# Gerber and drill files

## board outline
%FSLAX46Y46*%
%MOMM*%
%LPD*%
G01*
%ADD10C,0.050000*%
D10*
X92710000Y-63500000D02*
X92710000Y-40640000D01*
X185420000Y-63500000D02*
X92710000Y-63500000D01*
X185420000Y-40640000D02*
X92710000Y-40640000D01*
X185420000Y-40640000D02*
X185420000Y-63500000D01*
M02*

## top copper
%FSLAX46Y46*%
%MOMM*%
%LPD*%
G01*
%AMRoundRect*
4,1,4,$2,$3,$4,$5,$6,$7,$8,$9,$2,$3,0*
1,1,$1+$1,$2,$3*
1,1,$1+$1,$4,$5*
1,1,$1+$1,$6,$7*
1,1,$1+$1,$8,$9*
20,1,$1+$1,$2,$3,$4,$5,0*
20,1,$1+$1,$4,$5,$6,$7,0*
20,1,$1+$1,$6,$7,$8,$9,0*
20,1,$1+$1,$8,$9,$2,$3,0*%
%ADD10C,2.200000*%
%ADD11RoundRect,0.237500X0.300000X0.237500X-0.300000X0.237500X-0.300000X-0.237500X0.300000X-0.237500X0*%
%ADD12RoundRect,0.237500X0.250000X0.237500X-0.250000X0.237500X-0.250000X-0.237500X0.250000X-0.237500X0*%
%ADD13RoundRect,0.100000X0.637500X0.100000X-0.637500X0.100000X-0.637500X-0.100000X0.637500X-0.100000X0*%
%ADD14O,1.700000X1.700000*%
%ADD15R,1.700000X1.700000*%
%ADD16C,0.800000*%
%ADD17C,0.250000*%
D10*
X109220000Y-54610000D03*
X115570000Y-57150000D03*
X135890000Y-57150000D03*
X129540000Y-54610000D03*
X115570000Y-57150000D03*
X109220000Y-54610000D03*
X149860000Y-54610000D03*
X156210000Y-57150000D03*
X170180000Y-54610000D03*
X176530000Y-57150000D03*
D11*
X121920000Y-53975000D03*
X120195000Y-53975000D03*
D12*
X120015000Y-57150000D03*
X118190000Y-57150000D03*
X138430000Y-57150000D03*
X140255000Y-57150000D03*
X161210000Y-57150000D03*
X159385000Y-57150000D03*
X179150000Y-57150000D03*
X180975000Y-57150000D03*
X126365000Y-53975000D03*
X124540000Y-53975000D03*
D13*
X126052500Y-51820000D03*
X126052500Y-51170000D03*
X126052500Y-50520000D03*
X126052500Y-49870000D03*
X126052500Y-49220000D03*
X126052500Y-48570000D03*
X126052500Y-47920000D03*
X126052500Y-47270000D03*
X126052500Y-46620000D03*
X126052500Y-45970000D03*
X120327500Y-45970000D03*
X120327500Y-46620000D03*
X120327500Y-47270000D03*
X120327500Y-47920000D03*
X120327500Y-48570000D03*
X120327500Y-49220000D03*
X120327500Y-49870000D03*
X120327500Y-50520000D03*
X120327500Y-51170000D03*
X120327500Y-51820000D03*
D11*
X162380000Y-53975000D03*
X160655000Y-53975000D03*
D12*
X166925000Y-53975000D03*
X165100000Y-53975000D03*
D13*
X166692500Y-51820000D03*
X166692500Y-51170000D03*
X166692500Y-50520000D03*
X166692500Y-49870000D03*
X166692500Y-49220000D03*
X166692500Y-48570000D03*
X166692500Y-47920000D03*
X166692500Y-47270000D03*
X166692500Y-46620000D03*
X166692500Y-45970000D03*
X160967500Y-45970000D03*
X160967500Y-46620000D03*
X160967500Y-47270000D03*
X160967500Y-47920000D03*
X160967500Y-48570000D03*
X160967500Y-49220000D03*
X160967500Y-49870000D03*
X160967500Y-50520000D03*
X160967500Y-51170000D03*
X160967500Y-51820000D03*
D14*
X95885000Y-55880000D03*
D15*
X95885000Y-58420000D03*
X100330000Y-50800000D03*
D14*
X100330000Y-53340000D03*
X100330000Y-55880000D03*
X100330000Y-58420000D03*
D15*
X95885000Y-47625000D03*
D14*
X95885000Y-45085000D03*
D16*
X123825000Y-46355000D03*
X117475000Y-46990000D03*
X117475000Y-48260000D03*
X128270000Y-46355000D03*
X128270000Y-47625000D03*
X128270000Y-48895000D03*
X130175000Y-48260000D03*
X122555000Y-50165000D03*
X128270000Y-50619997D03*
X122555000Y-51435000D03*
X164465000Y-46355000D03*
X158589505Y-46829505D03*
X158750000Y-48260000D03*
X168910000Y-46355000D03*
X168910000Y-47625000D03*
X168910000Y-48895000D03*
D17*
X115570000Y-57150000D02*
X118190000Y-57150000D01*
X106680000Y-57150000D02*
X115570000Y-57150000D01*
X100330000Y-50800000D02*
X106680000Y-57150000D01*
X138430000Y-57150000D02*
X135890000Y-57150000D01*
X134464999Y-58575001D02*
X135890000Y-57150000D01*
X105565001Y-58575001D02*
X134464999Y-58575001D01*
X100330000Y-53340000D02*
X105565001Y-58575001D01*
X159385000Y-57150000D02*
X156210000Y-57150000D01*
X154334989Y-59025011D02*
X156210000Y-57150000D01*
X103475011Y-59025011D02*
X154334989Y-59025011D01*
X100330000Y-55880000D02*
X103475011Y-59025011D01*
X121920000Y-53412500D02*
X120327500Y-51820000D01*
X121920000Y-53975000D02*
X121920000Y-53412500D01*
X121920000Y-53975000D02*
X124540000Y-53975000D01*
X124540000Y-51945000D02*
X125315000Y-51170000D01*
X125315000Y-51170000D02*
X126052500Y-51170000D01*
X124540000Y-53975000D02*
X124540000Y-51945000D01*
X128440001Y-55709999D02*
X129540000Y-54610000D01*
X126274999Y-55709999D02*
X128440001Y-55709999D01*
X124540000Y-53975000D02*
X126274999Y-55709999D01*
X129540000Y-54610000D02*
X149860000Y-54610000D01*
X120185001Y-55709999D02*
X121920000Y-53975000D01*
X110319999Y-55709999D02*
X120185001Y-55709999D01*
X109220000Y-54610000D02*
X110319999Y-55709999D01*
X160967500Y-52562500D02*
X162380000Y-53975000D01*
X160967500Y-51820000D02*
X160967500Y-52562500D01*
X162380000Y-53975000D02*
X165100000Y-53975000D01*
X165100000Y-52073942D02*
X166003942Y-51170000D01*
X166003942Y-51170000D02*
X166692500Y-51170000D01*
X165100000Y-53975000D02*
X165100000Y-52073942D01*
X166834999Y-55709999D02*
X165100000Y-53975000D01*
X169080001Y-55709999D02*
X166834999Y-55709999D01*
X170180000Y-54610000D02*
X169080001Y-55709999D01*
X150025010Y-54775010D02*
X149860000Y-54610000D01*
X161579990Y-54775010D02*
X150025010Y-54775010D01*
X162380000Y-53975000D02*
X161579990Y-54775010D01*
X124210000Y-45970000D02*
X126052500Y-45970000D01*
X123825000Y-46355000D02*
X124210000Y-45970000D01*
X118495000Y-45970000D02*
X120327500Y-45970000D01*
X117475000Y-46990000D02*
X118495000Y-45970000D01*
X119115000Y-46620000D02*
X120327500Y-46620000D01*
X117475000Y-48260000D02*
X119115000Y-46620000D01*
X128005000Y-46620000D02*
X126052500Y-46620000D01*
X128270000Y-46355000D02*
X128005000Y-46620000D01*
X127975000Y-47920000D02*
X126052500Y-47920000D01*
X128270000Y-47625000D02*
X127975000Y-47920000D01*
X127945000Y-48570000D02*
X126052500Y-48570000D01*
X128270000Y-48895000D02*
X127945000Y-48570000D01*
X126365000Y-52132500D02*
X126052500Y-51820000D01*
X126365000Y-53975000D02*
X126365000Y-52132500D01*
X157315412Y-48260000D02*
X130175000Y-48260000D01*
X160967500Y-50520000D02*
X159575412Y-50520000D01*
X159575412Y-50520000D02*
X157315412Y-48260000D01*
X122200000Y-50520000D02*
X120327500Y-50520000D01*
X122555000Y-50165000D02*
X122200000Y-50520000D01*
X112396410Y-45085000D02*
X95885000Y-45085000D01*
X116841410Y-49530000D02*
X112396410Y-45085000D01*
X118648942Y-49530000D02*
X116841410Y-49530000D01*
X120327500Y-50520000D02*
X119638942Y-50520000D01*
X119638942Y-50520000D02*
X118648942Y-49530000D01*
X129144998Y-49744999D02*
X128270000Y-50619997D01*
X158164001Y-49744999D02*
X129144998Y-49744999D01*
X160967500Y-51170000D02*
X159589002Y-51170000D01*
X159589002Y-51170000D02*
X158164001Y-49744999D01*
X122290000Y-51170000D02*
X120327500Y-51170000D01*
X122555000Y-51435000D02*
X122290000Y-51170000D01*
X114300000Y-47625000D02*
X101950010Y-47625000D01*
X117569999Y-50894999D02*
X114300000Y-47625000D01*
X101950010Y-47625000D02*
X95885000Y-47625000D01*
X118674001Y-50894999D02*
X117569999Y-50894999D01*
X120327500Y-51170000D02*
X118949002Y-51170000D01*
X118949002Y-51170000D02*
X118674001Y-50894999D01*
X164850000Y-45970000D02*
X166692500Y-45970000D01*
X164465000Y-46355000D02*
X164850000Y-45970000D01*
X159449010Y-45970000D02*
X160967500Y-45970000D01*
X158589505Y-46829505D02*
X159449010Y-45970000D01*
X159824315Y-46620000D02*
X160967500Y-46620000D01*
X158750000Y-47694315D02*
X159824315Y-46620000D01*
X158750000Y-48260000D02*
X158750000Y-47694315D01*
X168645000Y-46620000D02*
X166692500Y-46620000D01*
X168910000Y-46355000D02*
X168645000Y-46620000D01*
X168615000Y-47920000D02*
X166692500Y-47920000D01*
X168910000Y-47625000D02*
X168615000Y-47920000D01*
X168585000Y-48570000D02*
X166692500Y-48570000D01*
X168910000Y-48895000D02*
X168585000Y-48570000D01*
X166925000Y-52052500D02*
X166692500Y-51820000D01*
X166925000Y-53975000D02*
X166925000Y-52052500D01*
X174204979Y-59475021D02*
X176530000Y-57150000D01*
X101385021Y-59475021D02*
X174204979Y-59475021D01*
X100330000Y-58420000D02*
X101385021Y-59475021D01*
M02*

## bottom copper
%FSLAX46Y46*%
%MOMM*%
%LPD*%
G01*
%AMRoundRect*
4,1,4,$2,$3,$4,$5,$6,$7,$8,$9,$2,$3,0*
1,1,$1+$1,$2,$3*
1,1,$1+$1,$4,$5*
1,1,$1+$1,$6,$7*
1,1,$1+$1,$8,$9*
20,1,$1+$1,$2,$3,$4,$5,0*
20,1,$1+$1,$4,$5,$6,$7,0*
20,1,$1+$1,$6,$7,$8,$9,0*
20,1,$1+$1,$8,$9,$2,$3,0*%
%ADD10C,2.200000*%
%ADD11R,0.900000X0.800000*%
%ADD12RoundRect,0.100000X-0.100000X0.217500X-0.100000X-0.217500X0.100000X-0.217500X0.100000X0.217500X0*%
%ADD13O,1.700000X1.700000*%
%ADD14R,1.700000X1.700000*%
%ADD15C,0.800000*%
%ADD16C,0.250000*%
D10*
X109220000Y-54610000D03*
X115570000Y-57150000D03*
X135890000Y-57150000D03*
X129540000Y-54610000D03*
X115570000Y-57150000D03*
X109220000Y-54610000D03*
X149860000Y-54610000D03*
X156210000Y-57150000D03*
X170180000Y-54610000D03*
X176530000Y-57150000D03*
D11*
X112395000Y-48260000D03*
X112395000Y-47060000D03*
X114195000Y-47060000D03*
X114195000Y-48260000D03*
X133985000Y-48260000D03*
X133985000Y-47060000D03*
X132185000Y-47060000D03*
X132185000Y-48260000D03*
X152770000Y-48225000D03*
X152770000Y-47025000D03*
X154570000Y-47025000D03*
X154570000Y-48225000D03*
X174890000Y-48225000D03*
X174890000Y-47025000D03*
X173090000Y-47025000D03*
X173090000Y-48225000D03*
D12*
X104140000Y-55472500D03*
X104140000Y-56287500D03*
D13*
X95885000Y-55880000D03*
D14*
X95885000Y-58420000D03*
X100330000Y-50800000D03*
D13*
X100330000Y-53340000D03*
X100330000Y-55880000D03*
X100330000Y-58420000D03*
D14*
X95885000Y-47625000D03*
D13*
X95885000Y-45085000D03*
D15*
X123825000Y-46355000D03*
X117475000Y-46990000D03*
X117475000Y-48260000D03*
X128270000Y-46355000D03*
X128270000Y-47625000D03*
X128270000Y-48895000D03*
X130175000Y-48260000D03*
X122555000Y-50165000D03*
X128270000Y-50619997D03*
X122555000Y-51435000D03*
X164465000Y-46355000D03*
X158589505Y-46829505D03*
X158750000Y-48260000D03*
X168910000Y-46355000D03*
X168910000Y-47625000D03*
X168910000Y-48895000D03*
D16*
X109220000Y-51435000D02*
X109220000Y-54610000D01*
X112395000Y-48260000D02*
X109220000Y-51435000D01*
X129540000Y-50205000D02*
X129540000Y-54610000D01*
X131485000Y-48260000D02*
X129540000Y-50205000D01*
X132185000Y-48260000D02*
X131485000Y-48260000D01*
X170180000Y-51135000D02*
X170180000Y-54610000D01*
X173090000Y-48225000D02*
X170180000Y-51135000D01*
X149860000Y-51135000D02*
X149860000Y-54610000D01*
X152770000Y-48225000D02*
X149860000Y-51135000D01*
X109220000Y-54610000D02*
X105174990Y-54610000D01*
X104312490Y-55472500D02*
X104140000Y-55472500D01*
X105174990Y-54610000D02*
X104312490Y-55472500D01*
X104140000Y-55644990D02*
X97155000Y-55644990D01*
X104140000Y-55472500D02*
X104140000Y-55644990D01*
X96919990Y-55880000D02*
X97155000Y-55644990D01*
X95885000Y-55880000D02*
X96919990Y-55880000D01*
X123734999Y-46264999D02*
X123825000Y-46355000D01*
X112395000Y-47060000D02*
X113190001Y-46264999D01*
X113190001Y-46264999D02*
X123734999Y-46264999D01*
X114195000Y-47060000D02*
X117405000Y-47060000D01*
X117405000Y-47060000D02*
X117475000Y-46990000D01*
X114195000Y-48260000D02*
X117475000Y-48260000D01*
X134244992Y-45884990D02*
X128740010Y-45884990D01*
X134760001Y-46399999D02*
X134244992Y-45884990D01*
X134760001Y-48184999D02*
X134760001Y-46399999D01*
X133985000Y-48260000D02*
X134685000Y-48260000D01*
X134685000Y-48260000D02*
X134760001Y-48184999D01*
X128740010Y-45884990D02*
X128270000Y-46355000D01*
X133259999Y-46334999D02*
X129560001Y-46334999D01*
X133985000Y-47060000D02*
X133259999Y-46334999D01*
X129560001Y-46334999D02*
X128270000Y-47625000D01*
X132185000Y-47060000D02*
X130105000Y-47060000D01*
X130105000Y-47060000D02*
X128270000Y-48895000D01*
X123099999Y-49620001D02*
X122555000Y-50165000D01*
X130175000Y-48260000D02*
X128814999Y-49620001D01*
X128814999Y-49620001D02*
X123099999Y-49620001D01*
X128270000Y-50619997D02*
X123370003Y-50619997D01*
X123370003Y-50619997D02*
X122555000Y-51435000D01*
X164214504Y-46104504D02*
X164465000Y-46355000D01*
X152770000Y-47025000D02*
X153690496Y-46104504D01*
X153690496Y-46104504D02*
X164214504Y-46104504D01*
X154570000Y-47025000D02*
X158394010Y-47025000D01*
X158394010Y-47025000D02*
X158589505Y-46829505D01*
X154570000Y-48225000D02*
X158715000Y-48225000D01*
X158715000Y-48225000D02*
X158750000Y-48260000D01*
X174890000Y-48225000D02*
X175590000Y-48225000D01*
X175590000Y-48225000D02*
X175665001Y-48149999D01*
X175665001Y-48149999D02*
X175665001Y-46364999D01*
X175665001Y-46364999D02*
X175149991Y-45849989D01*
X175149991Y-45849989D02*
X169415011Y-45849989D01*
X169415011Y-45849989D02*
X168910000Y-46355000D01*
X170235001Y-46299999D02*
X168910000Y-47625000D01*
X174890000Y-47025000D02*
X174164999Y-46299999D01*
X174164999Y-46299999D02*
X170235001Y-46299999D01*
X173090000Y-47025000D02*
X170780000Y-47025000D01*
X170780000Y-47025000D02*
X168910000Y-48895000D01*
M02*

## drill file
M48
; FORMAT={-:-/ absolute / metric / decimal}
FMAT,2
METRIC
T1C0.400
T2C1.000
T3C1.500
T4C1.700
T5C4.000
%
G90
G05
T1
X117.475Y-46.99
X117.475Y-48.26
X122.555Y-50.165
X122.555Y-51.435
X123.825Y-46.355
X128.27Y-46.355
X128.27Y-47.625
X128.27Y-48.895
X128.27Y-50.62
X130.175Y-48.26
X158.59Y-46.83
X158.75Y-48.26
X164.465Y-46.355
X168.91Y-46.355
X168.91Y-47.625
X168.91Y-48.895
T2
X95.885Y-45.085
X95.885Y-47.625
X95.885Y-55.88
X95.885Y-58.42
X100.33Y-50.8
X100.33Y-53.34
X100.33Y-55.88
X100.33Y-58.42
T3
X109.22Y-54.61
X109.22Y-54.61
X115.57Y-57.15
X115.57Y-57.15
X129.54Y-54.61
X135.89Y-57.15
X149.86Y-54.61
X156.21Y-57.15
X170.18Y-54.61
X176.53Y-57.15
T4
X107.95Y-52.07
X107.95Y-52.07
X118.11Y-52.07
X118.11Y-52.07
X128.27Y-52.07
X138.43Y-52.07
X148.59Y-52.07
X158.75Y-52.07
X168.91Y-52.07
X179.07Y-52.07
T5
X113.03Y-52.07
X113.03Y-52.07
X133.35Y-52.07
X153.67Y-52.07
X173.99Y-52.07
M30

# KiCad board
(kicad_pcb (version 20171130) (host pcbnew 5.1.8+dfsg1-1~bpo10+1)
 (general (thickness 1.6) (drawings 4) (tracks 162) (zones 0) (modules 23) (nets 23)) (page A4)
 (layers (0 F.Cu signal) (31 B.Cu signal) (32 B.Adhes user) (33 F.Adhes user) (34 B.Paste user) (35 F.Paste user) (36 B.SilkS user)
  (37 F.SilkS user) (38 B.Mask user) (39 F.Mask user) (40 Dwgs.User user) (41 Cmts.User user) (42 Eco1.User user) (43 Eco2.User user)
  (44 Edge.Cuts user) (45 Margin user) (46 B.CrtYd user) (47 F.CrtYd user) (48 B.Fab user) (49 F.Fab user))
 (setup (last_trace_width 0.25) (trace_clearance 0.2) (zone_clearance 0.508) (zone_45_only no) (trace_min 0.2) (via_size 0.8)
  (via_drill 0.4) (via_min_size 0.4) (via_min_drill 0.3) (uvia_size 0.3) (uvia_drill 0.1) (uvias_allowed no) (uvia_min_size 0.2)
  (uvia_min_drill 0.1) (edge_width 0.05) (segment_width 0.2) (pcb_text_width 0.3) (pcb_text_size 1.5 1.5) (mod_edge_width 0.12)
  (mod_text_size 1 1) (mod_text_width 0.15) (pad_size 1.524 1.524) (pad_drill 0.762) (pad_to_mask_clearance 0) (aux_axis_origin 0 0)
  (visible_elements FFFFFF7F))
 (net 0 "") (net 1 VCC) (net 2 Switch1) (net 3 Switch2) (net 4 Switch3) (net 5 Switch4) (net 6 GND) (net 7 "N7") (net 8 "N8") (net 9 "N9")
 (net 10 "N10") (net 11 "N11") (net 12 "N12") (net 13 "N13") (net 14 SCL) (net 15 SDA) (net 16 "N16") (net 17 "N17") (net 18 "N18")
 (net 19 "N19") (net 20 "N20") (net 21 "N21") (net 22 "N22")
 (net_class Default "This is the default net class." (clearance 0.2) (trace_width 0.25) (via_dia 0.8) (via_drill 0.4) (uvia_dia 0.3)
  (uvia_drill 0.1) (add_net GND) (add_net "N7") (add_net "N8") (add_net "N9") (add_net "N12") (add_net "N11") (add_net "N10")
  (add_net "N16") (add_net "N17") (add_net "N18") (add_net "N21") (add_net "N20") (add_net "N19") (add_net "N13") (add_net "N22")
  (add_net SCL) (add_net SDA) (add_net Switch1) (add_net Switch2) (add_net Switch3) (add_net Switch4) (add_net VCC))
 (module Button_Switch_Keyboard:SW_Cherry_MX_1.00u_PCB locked (layer B.Cu) (at 115.57 57.15)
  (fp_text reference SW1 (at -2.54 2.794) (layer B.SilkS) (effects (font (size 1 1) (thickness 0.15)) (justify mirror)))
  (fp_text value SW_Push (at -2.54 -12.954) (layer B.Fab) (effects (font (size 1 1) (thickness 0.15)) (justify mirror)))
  (pad "" np_thru_hole circle (at 2.54 -5.08) (size 1.7 1.7) (drill 1.7) (layers *.Cu *.Mask))
  (pad "" np_thru_hole circle (at -7.62 -5.08) (size 1.7 1.7) (drill 1.7) (layers *.Cu *.Mask))
  (pad "" np_thru_hole circle (at -2.54 -5.08) (size 4 4) (drill 4) (layers *.Cu *.Mask))
  (pad 2 thru_hole circle (at -6.35 -2.54) (size 2.2 2.2) (drill 1.5) (layers *.Cu *.Mask) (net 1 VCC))
  (pad 1 thru_hole circle (at 0 0) (size 2.2 2.2) (drill 1.5) (layers *.Cu *.Mask) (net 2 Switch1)))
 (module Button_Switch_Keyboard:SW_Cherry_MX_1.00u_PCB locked (layer B.Cu) (at 135.89 57.15)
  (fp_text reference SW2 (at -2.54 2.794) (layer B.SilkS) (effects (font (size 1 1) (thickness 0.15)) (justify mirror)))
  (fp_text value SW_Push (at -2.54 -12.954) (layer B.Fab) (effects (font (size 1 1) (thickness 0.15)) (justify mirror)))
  (pad 1 thru_hole circle (at 0 0) (size 2.2 2.2) (drill 1.5) (layers *.Cu *.Mask) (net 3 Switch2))
  (pad 2 thru_hole circle (at -6.35 -2.54) (size 2.2 2.2) (drill 1.5) (layers *.Cu *.Mask) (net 1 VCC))
  (pad "" np_thru_hole circle (at -2.54 -5.08) (size 4 4) (drill 4) (layers *.Cu *.Mask))
  (pad "" np_thru_hole circle (at -7.62 -5.08) (size 1.7 1.7) (drill 1.7) (layers *.Cu *.Mask))
  (pad "" np_thru_hole circle (at 2.54 -5.08) (size 1.7 1.7) (drill 1.7) (layers *.Cu *.Mask)))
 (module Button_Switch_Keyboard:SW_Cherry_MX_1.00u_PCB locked (layer B.Cu) (at 115.57 57.15)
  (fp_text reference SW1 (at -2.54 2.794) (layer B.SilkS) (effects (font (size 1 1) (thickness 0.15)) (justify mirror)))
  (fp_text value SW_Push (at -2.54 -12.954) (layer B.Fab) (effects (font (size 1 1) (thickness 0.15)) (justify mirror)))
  (pad 1 thru_hole circle (at 0 0) (size 2.2 2.2) (drill 1.5) (layers *.Cu *.Mask) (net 2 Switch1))
  (pad 2 thru_hole circle (at -6.35 -2.54) (size 2.2 2.2) (drill 1.5) (layers *.Cu *.Mask) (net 1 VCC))
  (pad "" np_thru_hole circle (at -2.54 -5.08) (size 4 4) (drill 4) (layers *.Cu *.Mask))
  (pad "" np_thru_hole circle (at -7.62 -5.08) (size 1.7 1.7) (drill 1.7) (layers *.Cu *.Mask))
  (pad "" np_thru_hole circle (at 2.54 -5.08) (size 1.7 1.7) (drill 1.7) (layers *.Cu *.Mask)))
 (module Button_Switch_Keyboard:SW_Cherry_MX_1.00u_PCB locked (layer B.Cu) (at 156.21 57.15)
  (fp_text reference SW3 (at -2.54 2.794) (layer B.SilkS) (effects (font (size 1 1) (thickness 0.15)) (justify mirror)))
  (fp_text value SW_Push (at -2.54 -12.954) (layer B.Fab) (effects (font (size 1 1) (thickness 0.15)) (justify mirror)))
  (pad "" np_thru_hole circle (at 2.54 -5.08) (size 1.7 1.7) (drill 1.7) (layers *.Cu *.Mask))
  (pad "" np_thru_hole circle (at -7.62 -5.08) (size 1.7 1.7) (drill 1.7) (layers *.Cu *.Mask))
  (pad "" np_thru_hole circle (at -2.54 -5.08) (size 4 4) (drill 4) (layers *.Cu *.Mask))
  (pad 2 thru_hole circle (at -6.35 -2.54) (size 2.2 2.2) (drill 1.5) (layers *.Cu *.Mask) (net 1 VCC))
  (pad 1 thru_hole circle (at 0 0) (size 2.2 2.2) (drill 1.5) (layers *.Cu *.Mask) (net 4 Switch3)))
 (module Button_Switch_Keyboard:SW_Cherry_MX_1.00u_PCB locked (layer B.Cu) (at 176.53 57.15)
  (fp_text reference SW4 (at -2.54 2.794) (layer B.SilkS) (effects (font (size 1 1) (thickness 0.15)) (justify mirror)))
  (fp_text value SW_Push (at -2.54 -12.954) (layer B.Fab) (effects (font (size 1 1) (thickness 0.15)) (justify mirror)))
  (pad "" np_thru_hole circle (at 2.54 -5.08) (size 1.7 1.7) (drill 1.7) (layers *.Cu *.Mask))
  (pad "" np_thru_hole circle (at -7.62 -5.08) (size 1.7 1.7) (drill 1.7) (layers *.Cu *.Mask))
  (pad "" np_thru_hole circle (at -2.54 -5.08) (size 4 4) (drill 4) (layers *.Cu *.Mask))
  (pad 2 thru_hole circle (at -6.35 -2.54) (size 2.2 2.2) (drill 1.5) (layers *.Cu *.Mask) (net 1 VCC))
  (pad 1 thru_hole circle (at 0 0) (size 2.2 2.2) (drill 1.5) (layers *.Cu *.Mask) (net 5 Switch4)))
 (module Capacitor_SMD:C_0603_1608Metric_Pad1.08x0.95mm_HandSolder (layer F.Cu) (at 121.0575 53.975 180)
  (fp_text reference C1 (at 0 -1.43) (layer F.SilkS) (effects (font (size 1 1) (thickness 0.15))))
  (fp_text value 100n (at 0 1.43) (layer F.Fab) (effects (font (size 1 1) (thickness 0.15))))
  (pad 1 smd roundrect (at -0.8625 0 180) (size 1.075 0.95) (layers F.Cu F.Paste F.Mask) (roundrect_rratio 0.25) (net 1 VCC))
  (pad 2 smd roundrect (at 0.8625 0 180) (size 1.075 0.95) (layers F.Cu F.Paste F.Mask) (roundrect_rratio 0.25) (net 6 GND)))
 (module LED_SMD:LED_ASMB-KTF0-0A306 (layer B.Cu) (at 113.295 47.66)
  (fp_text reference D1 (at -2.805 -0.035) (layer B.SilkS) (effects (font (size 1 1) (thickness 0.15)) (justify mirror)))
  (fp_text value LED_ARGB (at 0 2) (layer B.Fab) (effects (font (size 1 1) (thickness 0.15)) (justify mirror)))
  (pad 1 smd rect (at -0.9 0.6) (size 0.9 0.8) (layers B.Cu B.Paste B.Mask) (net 1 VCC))
  (pad 2 smd rect (at -0.9 -0.6) (size 0.9 0.8) (layers B.Cu B.Paste B.Mask) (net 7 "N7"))
  (pad 3 smd rect (at 0.9 -0.6) (size 0.9 0.8) (layers B.Cu B.Paste B.Mask) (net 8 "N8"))
  (pad 4 smd rect (at 0.9 0.6) (size 0.9 0.8) (layers B.Cu B.Paste B.Mask) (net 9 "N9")))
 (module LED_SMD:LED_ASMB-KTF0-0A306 (layer B.Cu) (at 133.085 47.66)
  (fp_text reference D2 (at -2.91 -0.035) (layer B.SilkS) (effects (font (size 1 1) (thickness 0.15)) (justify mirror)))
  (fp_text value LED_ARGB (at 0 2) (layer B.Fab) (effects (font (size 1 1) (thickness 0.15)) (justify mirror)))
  (pad 4 smd rect (at 0.9 0.6) (size 0.9 0.8) (layers B.Cu B.Paste B.Mask) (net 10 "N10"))
  (pad 3 smd rect (at 0.9 -0.6) (size 0.9 0.8) (layers B.Cu B.Paste B.Mask) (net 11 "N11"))
  (pad 2 smd rect (at -0.9 -0.6) (size 0.9 0.8) (layers B.Cu B.Paste B.Mask) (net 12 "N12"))
  (pad 1 smd rect (at -0.9 0.6) (size 0.9 0.8) (layers B.Cu B.Paste B.Mask) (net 1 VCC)))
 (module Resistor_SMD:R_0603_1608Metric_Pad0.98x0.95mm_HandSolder (layer F.Cu) (at 119.1025 57.15 180)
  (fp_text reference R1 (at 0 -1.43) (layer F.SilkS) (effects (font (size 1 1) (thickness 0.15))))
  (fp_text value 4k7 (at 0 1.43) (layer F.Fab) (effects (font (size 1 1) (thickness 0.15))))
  (pad 1 smd roundrect (at -0.9125 0 180) (size 0.975 0.95) (layers F.Cu F.Paste F.Mask) (roundrect_rratio 0.25) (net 6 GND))
  (pad 2 smd roundrect (at 0.9125 0 180) (size 0.975 0.95) (layers F.Cu F.Paste F.Mask) (roundrect_rratio 0.25) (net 2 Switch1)))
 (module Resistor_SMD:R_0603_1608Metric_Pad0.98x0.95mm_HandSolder (layer F.Cu) (at 139.3425 57.15 180)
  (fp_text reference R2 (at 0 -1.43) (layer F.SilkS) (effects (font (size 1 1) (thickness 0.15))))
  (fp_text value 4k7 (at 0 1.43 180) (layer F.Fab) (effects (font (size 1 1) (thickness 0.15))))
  (pad 2 smd roundrect (at 0.9125 0 180) (size 0.975 0.95) (layers F.Cu F.Paste F.Mask) (roundrect_rratio 0.25) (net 3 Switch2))
  (pad 1 smd roundrect (at -0.9125 0 180) (size 0.975 0.95) (layers F.Cu F.Paste F.Mask) (roundrect_rratio 0.25) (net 6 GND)))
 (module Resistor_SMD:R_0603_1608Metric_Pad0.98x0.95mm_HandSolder (layer F.Cu) (at 160.2975 57.15 180)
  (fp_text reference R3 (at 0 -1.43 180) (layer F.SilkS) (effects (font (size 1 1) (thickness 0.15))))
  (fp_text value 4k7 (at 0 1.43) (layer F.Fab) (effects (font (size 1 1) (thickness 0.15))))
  (pad 1 smd roundrect (at -0.9125 0 180) (size 0.975 0.95) (layers F.Cu F.Paste F.Mask) (roundrect_rratio 0.25) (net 6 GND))
  (pad 2 smd roundrect (at 0.9125 0 180) (size 0.975 0.95) (layers F.Cu F.Paste F.Mask) (roundrect_rratio 0.25) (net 4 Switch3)))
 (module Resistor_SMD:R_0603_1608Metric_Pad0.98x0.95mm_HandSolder (layer F.Cu) (at 180.0625 57.15 180)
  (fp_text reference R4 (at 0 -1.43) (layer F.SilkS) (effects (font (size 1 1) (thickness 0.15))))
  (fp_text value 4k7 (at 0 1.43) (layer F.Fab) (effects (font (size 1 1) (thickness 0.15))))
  (pad 2 smd roundrect (at 0.9125 0 180) (size 0.975 0.95) (layers F.Cu F.Paste F.Mask) (roundrect_rratio 0.25))
  (pad 1 smd roundrect (at -0.9125 0 180) (size 0.975 0.95) (layers F.Cu F.Paste F.Mask) (roundrect_rratio 0.25) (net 6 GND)))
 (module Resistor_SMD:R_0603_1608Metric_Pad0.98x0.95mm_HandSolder (layer F.Cu) (at 125.4525 53.975 180)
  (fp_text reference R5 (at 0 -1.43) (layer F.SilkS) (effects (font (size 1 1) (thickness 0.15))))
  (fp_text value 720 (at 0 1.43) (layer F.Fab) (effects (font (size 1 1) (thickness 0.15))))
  (pad 1 smd roundrect (at -0.9125 0 180) (size 0.975 0.95) (layers F.Cu F.Paste F.Mask) (roundrect_rratio 0.25) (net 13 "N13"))
  (pad 2 smd roundrect (at 0.9125 0 180) (size 0.975 0.95) (layers F.Cu F.Paste F.Mask) (roundrect_rratio 0.25) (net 1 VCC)))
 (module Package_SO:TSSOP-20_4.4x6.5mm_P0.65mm (layer F.Cu) (at 123.19 48.895 180)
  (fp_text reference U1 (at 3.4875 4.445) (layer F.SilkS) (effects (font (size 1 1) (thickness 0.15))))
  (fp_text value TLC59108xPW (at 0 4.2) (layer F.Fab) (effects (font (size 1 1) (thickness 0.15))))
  (pad 1 smd roundrect (at -2.8625 -2.925 180) (size 1.475 0.4) (layers F.Cu F.Paste F.Mask) (roundrect_rratio 0.25) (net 13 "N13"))
  (pad 2 smd roundrect (at -2.8625 -2.275 180) (size 1.475 0.4) (layers F.Cu F.Paste F.Mask) (roundrect_rratio 0.25) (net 1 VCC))
  (pad 3 smd roundrect (at -2.8625 -1.625 180) (size 1.475 0.4) (layers F.Cu F.Paste F.Mask) (roundrect_rratio 0.25) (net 6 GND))
  (pad 4 smd roundrect (at -2.8625 -0.975 180) (size 1.475 0.4) (layers F.Cu F.Paste F.Mask) (roundrect_rratio 0.25) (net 6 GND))
  (pad 5 smd roundrect (at -2.8625 -0.325 180) (size 1.475 0.4) (layers F.Cu F.Paste F.Mask) (roundrect_rratio 0.25) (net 6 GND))
  (pad 6 smd roundrect (at -2.8625 0.325 180) (size 1.475 0.4) (layers F.Cu F.Paste F.Mask) (roundrect_rratio 0.25) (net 12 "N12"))
  (pad 7 smd roundrect (at -2.8625 0.975 180) (size 1.475 0.4) (layers F.Cu F.Paste F.Mask) (roundrect_rratio 0.25) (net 11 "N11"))
  (pad 8 smd roundrect (at -2.8625 1.625 180) (size 1.475 0.4) (layers F.Cu F.Paste F.Mask) (roundrect_rratio 0.25) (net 6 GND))
  (pad 9 smd roundrect (at -2.8625 2.275 180) (size 1.475 0.4) (layers F.Cu F.Paste F.Mask) (roundrect_rratio 0.25) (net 10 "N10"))
  (pad 10 smd roundrect (at -2.8625 2.925 180) (size 1.475 0.4) (layers F.Cu F.Paste F.Mask) (roundrect_rratio 0.25) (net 7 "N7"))
  (pad 11 smd roundrect (at 2.8625 2.925 180) (size 1.475 0.4) (layers F.Cu F.Paste F.Mask) (roundrect_rratio 0.25) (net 8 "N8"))
  (pad 12 smd roundrect (at 2.8625 2.275 180) (size 1.475 0.4) (layers F.Cu F.Paste F.Mask) (roundrect_rratio 0.25) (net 9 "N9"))
  (pad 13 smd roundrect (at 2.8625 1.625 180) (size 1.475 0.4) (layers F.Cu F.Paste F.Mask) (roundrect_rratio 0.25) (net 6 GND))
  (pad 14 smd roundrect (at 2.8625 0.975 180) (size 1.475 0.4) (layers F.Cu F.Paste F.Mask) (roundrect_rratio 0.25))
  (pad 15 smd roundrect (at 2.8625 0.325 180) (size 1.475 0.4) (layers F.Cu F.Paste F.Mask) (roundrect_rratio 0.25))
  (pad 16 smd roundrect (at 2.8625 -0.325 180) (size 1.475 0.4) (layers F.Cu F.Paste F.Mask) (roundrect_rratio 0.25) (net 6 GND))
  (pad 17 smd roundrect (at 2.8625 -0.975 180) (size 1.475 0.4) (layers F.Cu F.Paste F.Mask) (roundrect_rratio 0.25) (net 1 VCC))
  (pad 18 smd roundrect (at 2.8625 -1.625 180) (size 1.475 0.4) (layers F.Cu F.Paste F.Mask) (roundrect_rratio 0.25) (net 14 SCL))
  (pad 19 smd roundrect (at 2.8625 -2.275 180) (size 1.475 0.4) (layers F.Cu F.Paste F.Mask) (roundrect_rratio 0.25) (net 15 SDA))
  (pad 20 smd roundrect (at 2.8625 -2.925 180) (size 1.475 0.4) (layers F.Cu F.Paste F.Mask) (roundrect_rratio 0.25) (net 1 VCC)))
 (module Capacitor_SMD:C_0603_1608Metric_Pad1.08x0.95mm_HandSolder (layer F.Cu) (at 161.5175 53.975 180)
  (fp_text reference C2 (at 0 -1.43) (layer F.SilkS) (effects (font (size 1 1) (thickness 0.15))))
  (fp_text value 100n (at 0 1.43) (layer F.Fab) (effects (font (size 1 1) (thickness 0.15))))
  (pad 1 smd roundrect (at -0.8625 0 180) (size 1.075 0.95) (layers F.Cu F.Paste F.Mask) (roundrect_rratio 0.25) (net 1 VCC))
  (pad 2 smd roundrect (at 0.8625 0 180) (size 1.075 0.95) (layers F.Cu F.Paste F.Mask) (roundrect_rratio 0.25) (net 6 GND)))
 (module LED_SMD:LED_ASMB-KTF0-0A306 (layer B.Cu) (at 153.67 47.625)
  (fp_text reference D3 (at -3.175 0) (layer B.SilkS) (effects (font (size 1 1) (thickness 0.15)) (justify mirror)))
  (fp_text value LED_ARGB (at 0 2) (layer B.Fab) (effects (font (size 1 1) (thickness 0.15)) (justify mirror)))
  (pad 1 smd rect (at -0.9 0.6) (size 0.9 0.8) (layers B.Cu B.Paste B.Mask) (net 1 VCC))
  (pad 2 smd rect (at -0.9 -0.6) (size 0.9 0.8) (layers B.Cu B.Paste B.Mask) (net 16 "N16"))
  (pad 3 smd rect (at 0.9 -0.6) (size 0.9 0.8) (layers B.Cu B.Paste B.Mask) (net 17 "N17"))
  (pad 4 smd rect (at 0.9 0.6) (size 0.9 0.8) (layers B.Cu B.Paste B.Mask) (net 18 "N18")))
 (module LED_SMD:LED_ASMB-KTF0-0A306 (layer B.Cu) (at 173.99 47.625)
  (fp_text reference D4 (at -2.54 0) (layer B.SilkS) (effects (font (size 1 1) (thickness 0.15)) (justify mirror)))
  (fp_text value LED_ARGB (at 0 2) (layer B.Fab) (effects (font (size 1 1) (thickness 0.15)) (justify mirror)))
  (pad 4 smd rect (at 0.9 0.6) (size 0.9 0.8) (layers B.Cu B.Paste B.Mask) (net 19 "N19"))
  (pad 3 smd rect (at 0.9 -0.6) (size 0.9 0.8) (layers B.Cu B.Paste B.Mask) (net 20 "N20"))
  (pad 2 smd rect (at -0.9 -0.6) (size 0.9 0.8) (layers B.Cu B.Paste B.Mask) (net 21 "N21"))
  (pad 1 smd rect (at -0.9 0.6) (size 0.9 0.8) (layers B.Cu B.Paste B.Mask) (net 1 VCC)))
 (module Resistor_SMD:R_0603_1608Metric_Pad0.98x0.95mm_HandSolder (layer F.Cu) (at 166.0125 53.975 180)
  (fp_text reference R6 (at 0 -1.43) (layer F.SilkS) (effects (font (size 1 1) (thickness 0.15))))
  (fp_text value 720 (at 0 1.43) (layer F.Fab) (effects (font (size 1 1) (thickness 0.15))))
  (pad 1 smd roundrect (at -0.9125 0 180) (size 0.975 0.95) (layers F.Cu F.Paste F.Mask) (roundrect_rratio 0.25) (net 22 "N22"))
  (pad 2 smd roundrect (at 0.9125 0 180) (size 0.975 0.95) (layers F.Cu F.Paste F.Mask) (roundrect_rratio 0.25) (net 1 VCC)))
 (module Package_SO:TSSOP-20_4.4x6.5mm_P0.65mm (layer F.Cu) (at 163.83 48.895 180)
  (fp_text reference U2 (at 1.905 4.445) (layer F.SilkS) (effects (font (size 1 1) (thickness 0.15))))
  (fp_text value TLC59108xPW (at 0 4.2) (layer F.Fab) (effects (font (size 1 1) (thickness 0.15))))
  (pad 1 smd roundrect (at -2.8625 -2.925 180) (size 1.475 0.4) (layers F.Cu F.Paste F.Mask) (roundrect_rratio 0.25) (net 22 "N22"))
  (pad 2 smd roundrect (at -2.8625 -2.275 180) (size 1.475 0.4) (layers F.Cu F.Paste F.Mask) (roundrect_rratio 0.25) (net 1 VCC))
  (pad 3 smd roundrect (at -2.8625 -1.625 180) (size 1.475 0.4) (layers F.Cu F.Paste F.Mask) (roundrect_rratio 0.25) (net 1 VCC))
  (pad 4 smd roundrect (at -2.8625 -0.975 180) (size 1.475 0.4) (layers F.Cu F.Paste F.Mask) (roundrect_rratio 0.25) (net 6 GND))
  (pad 5 smd roundrect (at -2.8625 -0.325 180) (size 1.475 0.4) (layers F.Cu F.Paste F.Mask) (roundrect_rratio 0.25) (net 6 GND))
  (pad 6 smd roundrect (at -2.8625 0.325 180) (size 1.475 0.4) (layers F.Cu F.Paste F.Mask) (roundrect_rratio 0.25) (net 21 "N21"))
  (pad 7 smd roundrect (at -2.8625 0.975 180) (size 1.475 0.4) (layers F.Cu F.Paste F.Mask) (roundrect_rratio 0.25) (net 20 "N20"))
  (pad 8 smd roundrect (at -2.8625 1.625 180) (size 1.475 0.4) (layers F.Cu F.Paste F.Mask) (roundrect_rratio 0.25) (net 6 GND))
  (pad 9 smd roundrect (at -2.8625 2.275 180) (size 1.475 0.4) (layers F.Cu F.Paste F.Mask) (roundrect_rratio 0.25) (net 19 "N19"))
  (pad 10 smd roundrect (at -2.8625 2.925 180) (size 1.475 0.4) (layers F.Cu F.Paste F.Mask) (roundrect_rratio 0.25) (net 16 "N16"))
  (pad 11 smd roundrect (at 2.8625 2.925 180) (size 1.475 0.4) (layers F.Cu F.Paste F.Mask) (roundrect_rratio 0.25) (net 17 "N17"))
  (pad 12 smd roundrect (at 2.8625 2.275 180) (size 1.475 0.4) (layers F.Cu F.Paste F.Mask) (roundrect_rratio 0.25) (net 18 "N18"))
  (pad 13 smd roundrect (at 2.8625 1.625 180) (size 1.475 0.4) (layers F.Cu F.Paste F.Mask) (roundrect_rratio 0.25) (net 6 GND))
  (pad 14 smd roundrect (at 2.8625 0.975 180) (size 1.475 0.4) (layers F.Cu F.Paste F.Mask) (roundrect_rratio 0.25))
  (pad 15 smd roundrect (at 2.8625 0.325 180) (size 1.475 0.4) (layers F.Cu F.Paste F.Mask) (roundrect_rratio 0.25))
  (pad 16 smd roundrect (at 2.8625 -0.325 180) (size 1.475 0.4) (layers F.Cu F.Paste F.Mask) (roundrect_rratio 0.25) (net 6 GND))
  (pad 17 smd roundrect (at 2.8625 -0.975 180) (size 1.475 0.4) (layers F.Cu F.Paste F.Mask) (roundrect_rratio 0.25) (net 1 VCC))
  (pad 18 smd roundrect (at 2.8625 -1.625 180) (size 1.475 0.4) (layers F.Cu F.Paste F.Mask) (roundrect_rratio 0.25) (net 14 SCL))
  (pad 19 smd roundrect (at 2.8625 -2.275 180) (size 1.475 0.4) (layers F.Cu F.Paste F.Mask) (roundrect_rratio 0.25) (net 15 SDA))
  (pad 20 smd roundrect (at 2.8625 -2.925 180) (size 1.475 0.4) (layers F.Cu F.Paste F.Mask) (roundrect_rratio 0.25) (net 1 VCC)))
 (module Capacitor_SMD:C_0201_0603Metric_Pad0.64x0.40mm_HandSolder (layer B.Cu) (at 104.14 55.88 270)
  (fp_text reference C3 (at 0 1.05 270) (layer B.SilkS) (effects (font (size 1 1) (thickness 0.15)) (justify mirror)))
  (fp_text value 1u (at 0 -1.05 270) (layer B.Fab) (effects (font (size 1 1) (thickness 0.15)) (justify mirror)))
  (pad "" smd roundrect (at -0.4325 0 270) (size 0.458 0.36) (layers B.Paste) (roundrect_rratio 0.25))
  (pad "" smd roundrect (at 0.4325 0 270) (size 0.458 0.36) (layers B.Paste) (roundrect_rratio 0.25))
  (pad 1 smd roundrect (at -0.4075 0 270) (size 0.635 0.4) (layers B.Cu B.Mask) (roundrect_rratio 0.25) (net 1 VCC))
  (pad 2 smd roundrect (at 0.4075 0 270) (size 0.635 0.4) (layers B.Cu B.Mask) (roundrect_rratio 0.25) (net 6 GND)))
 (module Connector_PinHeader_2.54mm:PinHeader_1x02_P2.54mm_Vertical (layer F.Cu) (at 95.885 58.42 180)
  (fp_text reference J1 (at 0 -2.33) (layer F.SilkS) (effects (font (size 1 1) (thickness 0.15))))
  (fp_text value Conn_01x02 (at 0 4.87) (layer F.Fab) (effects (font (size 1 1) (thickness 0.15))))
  (pad 2 thru_hole oval (at 0 2.54 180) (size 1.7 1.7) (drill 1) (layers *.Cu *.Mask) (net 1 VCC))
  (pad 1 thru_hole rect (at 0 0 180) (size 1.7 1.7) (drill 1) (layers *.Cu *.Mask) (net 6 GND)))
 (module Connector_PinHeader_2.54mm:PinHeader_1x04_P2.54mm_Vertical (layer B.Cu) (at 100.33 50.8 180)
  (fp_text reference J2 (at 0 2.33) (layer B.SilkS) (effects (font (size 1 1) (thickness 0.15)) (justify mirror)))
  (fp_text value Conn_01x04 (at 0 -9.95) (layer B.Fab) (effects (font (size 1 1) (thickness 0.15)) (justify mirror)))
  (pad 1 thru_hole rect (at 0 0 180) (size 1.7 1.7) (drill 1) (layers *.Cu *.Mask) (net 2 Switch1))
  (pad 2 thru_hole oval (at 0 -2.54 180) (size 1.7 1.7) (drill 1) (layers *.Cu *.Mask) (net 3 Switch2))
  (pad 3 thru_hole oval (at 0 -5.08 180) (size 1.7 1.7) (drill 1) (layers *.Cu *.Mask) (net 4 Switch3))
  (pad 4 thru_hole oval (at 0 -7.62 180) (size 1.7 1.7) (drill 1) (layers *.Cu *.Mask) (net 5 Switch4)))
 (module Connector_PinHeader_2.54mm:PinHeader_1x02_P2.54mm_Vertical (layer B.Cu) (at 95.885 47.625)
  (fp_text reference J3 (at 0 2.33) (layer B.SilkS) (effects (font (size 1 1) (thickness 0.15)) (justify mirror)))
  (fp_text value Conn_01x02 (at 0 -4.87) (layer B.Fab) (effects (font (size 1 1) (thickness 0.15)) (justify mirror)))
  (pad 1 thru_hole rect (at 0 0) (size 1.7 1.7) (drill 1) (layers *.Cu *.Mask) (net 15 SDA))
  (pad 2 thru_hole oval (at 0 -2.54) (size 1.7 1.7) (drill 1) (layers *.Cu *.Mask) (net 14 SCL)))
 (gr_line (start 92.71 63.5) (end 92.71 40.64) (layer Edge.Cuts) (width 0.05))
 (gr_line (start 185.42 63.5) (end 92.71 63.5) (layer Edge.Cuts) (width 0.05))
 (gr_line (start 185.42 40.64) (end 92.71 40.64) (layer Edge.Cuts) (width 0.05))
 (gr_line (start 185.42 40.64) (end 185.42 63.5) (layer Edge.Cuts) (width 0.05))
 (segment (start 115.57 57.15) (end 118.19 57.15) (width 0.25) (layer F.Cu) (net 2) (status 30))
 (segment (start 106.68 57.15) (end 115.57 57.15) (width 0.25) (layer F.Cu) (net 2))
 (segment (start 100.33 50.8) (end 106.68 57.15) (width 0.25) (layer F.Cu) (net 2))
 (segment (start 138.43 57.15) (end 135.89 57.15) (width 0.25) (layer F.Cu) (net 3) (status 30))
 (segment (start 134.464999 58.575001) (end 135.89 57.15) (width 0.25) (layer F.Cu) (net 3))
 (segment (start 105.565001 58.575001) (end 134.464999 58.575001) (width 0.25) (layer F.Cu) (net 3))
 (segment (start 100.33 53.34) (end 105.565001 58.575001) (width 0.25) (layer F.Cu) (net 3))
 (segment (start 159.385 57.15) (end 156.21 57.15) (width 0.25) (layer F.Cu) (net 4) (status 30))
 (segment (start 154.334989 59.025011) (end 156.21 57.15) (width 0.25) (layer F.Cu) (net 4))
 (segment (start 103.475011 59.025011) (end 154.334989 59.025011) (width 0.25) (layer F.Cu) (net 4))
 (segment (start 100.33 55.88) (end 103.475011 59.025011) (width 0.25) (layer F.Cu) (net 4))
 (segment (start 121.92 53.4125) (end 120.3275 51.82) (width 0.25) (layer F.Cu) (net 1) (status 20))
 (segment (start 121.92 53.975) (end 121.92 53.4125) (width 0.25) (layer F.Cu) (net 1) (status 10))
 (segment (start 121.92 53.975) (end 124.54 53.975) (width 0.25) (layer F.Cu) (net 1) (status 30))
 (segment (start 124.54 51.945) (end 125.315 51.17) (width 0.25) (layer F.Cu) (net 1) (status 20))
 (segment (start 125.315 51.17) (end 126.0525 51.17) (width 0.25) (layer F.Cu) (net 1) (status 30))
 (segment (start 124.54 53.975) (end 124.54 51.945) (width 0.25) (layer F.Cu) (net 1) (status 10))
 (segment (start 128.440001 55.709999) (end 129.54 54.61) (width 0.25) (layer F.Cu) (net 1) (status 20))
 (segment (start 126.274999 55.709999) (end 128.440001 55.709999) (width 0.25) (layer F.Cu) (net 1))
 (segment (start 124.54 53.975) (end 126.274999 55.709999) (width 0.25) (layer F.Cu) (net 1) (status 10))
 (segment (start 129.54 54.61) (end 149.86 54.61) (width 0.25) (layer F.Cu) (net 1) (status 30))
 (segment (start 120.185001 55.709999) (end 121.92 53.975) (width 0.25) (layer F.Cu) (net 1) (status 20))
 (segment (start 110.319999 55.709999) (end 120.185001 55.709999) (width 0.25) (layer F.Cu) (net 1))
 (segment (start 109.22 54.61) (end 110.319999 55.709999) (width 0.25) (layer F.Cu) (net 1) (status 10))
 (segment (start 109.22 51.435) (end 109.22 54.61) (width 0.25) (layer B.Cu) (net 1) (status 20))
 (segment (start 112.395 48.26) (end 109.22 51.435) (width 0.25) (layer B.Cu) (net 1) (status 10))
 (segment (start 129.54 50.205) (end 129.54 54.61) (width 0.25) (layer B.Cu) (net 1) (status 20))
 (segment (start 131.485 48.26) (end 129.54 50.205) (width 0.25) (layer B.Cu) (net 1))
 (segment (start 132.185 48.26) (end 131.485 48.26) (width 0.25) (layer B.Cu) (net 1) (status 10))
 (segment (start 160.9675 52.5625) (end 162.38 53.975) (width 0.25) (layer F.Cu) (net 1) (status 20))
 (segment (start 160.9675 51.82) (end 160.9675 52.5625) (width 0.25) (layer F.Cu) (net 1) (status 10))
 (segment (start 162.38 53.975) (end 165.1 53.975) (width 0.25) (layer F.Cu) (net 1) (status 30))
 (segment (start 165.1 52.073942) (end 166.003942 51.17) (width 0.25) (layer F.Cu) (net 1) (status 20))
 (segment (start 166.003942 51.17) (end 166.6925 51.17) (width 0.25) (layer F.Cu) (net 1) (status 30))
 (segment (start 165.1 53.975) (end 165.1 52.073942) (width 0.25) (layer F.Cu) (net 1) (status 10))
 (segment (start 166.834999 55.709999) (end 165.1 53.975) (width 0.25) (layer F.Cu) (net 1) (status 20))
 (segment (start 169.080001 55.709999) (end 166.834999 55.709999) (width 0.25) (layer F.Cu) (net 1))
 (segment (start 170.18 54.61) (end 169.080001 55.709999) (width 0.25) (layer F.Cu) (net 1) (status 10))
 (segment (start 150.02501 54.77501) (end 149.86 54.61) (width 0.25) (layer F.Cu) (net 1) (status 30))
 (segment (start 161.57999 54.77501) (end 150.02501 54.77501) (width 0.25) (layer F.Cu) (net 1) (status 20))
 (segment (start 162.38 53.975) (end 161.57999 54.77501) (width 0.25) (layer F.Cu) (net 1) (status 10))
 (segment (start 170.18 51.135) (end 170.18 54.61) (width 0.25) (layer B.Cu) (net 1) (status 20))
 (segment (start 173.09 48.225) (end 170.18 51.135) (width 0.25) (layer B.Cu) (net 1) (status 10))
 (segment (start 149.86 51.135) (end 149.86 54.61) (width 0.25) (layer B.Cu) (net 1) (status 20))
 (segment (start 152.77 48.225) (end 149.86 51.135) (width 0.25) (layer B.Cu) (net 1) (status 10))
 (segment (start 109.22 54.61) (end 105.17499 54.61) (width 0.25) (layer B.Cu) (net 1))
 (segment (start 104.31249 55.4725) (end 104.14 55.4725) (width 0.25) (layer B.Cu) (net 1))
 (segment (start 105.17499 54.61) (end 104.31249 55.4725) (width 0.25) (layer B.Cu) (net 1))
 (segment (start 104.14 55.64499) (end 97.155 55.64499) (width 0.25) (layer B.Cu) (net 1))
 (segment (start 104.14 55.4725) (end 104.14 55.64499) (width 0.25) (layer B.Cu) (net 1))
 (segment (start 96.91999 55.88) (end 97.155 55.64499) (width 0.25) (layer B.Cu) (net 1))
 (segment (start 95.885 55.88) (end 96.91999 55.88) (width 0.25) (layer B.Cu) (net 1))
 (via (at 123.825 46.355) (size 0.8) (drill 0.4) (layers F.Cu B.Cu) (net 7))
 (segment (start 123.734999 46.264999) (end 123.825 46.355) (width 0.25) (layer B.Cu) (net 7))
 (segment (start 112.395 47.06) (end 113.190001 46.264999) (width 0.25) (layer B.Cu) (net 7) (status 10))
 (segment (start 113.190001 46.264999) (end 123.734999 46.264999) (width 0.25) (layer B.Cu) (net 7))
 (segment (start 124.21 45.97) (end 126.0525 45.97) (width 0.25) (layer F.Cu) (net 7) (status 20))
 (segment (start 123.825 46.355) (end 124.21 45.97) (width 0.25) (layer F.Cu) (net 7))
 (segment (start 114.195 47.06) (end 117.405 47.06) (width 0.25) (layer B.Cu) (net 8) (status 10))
 (via (at 117.475 46.99) (size 0.8) (drill 0.4) (layers F.Cu B.Cu) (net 8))
 (segment (start 117.405 47.06) (end 117.475 46.99) (width 0.25) (layer B.Cu) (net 8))
 (segment (start 118.495 45.97) (end 120.3275 45.97) (width 0.25) (layer F.Cu) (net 8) (status 20))
 (segment (start 117.475 46.99) (end 118.495 45.97) (width 0.25) (layer F.Cu) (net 8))
 (via (at 117.475 48.26) (size 0.8) (drill 0.4) (layers F.Cu B.Cu) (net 9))
 (segment (start 114.195 48.26) (end 117.475 48.26) (width 0.25) (layer B.Cu) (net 9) (status 10))
 (segment (start 119.115 46.62) (end 120.3275 46.62) (width 0.25) (layer F.Cu) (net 9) (status 20))
 (segment (start 117.475 48.26) (end 119.115 46.62) (width 0.25) (layer F.Cu) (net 9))
 (segment (start 134.244992 45.88499) (end 128.74001 45.88499) (width 0.25) (layer B.Cu) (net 10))
 (segment (start 134.760001 46.399999) (end 134.244992 45.88499) (width 0.25) (layer B.Cu) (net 10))
 (segment (start 134.760001 48.184999) (end 134.760001 46.399999) (width 0.25) (layer B.Cu) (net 10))
 (segment (start 133.985 48.26) (end 134.685 48.26) (width 0.25) (layer B.Cu) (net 10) (status 10))
 (segment (start 134.685 48.26) (end 134.760001 48.184999) (width 0.25) (layer B.Cu) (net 10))
 (via (at 128.27 46.355) (size 0.8) (drill 0.4) (layers F.Cu B.Cu) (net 10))
 (segment (start 128.74001 45.88499) (end 128.27 46.355) (width 0.25) (layer B.Cu) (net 10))
 (segment (start 128.005 46.62) (end 126.0525 46.62) (width 0.25) (layer F.Cu) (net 10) (status 20))
 (segment (start 128.27 46.355) (end 128.005 46.62) (width 0.25) (layer F.Cu) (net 10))
 (segment (start 133.259999 46.334999) (end 129.560001 46.334999) (width 0.25) (layer B.Cu) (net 11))
 (segment (start 133.985 47.06) (end 133.259999 46.334999) (width 0.25) (layer B.Cu) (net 11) (status 10))
 (via (at 128.27 47.625) (size 0.8) (drill 0.4) (layers F.Cu B.Cu) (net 11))
 (segment (start 129.560001 46.334999) (end 128.27 47.625) (width 0.25) (layer B.Cu) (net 11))
 (segment (start 127.975 47.92) (end 126.0525 47.92) (width 0.25) (layer F.Cu) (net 11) (status 20))
 (segment (start 128.27 47.625) (end 127.975 47.92) (width 0.25) (layer F.Cu) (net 11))
 (segment (start 132.185 47.06) (end 130.105 47.06) (width 0.25) (layer B.Cu) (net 12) (status 10))
 (via (at 128.27 48.895) (size 0.8) (drill 0.4) (layers F.Cu B.Cu) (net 12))
 (segment (start 130.105 47.06) (end 128.27 48.895) (width 0.25) (layer B.Cu) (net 12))
 (segment (start 127.945 48.57) (end 126.0525 48.57) (width 0.25) (layer F.Cu) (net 12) (status 20))
 (segment (start 128.27 48.895) (end 127.945 48.57) (width 0.25) (layer F.Cu) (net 12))
 (segment (start 126.365 52.1325) (end 126.0525 51.82) (width 0.25) (layer F.Cu) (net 13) (status 20))
 (segment (start 126.365 53.975) (end 126.365 52.1325) (width 0.25) (layer F.Cu) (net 13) (status 10))
 (via (at 130.175 48.26) (size 0.8) (drill 0.4) (layers F.Cu B.Cu) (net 14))
 (segment (start 157.315412 48.26) (end 130.175 48.26) (width 0.25) (layer F.Cu) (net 14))
 (segment (start 160.9675 50.52) (end 159.575412 50.52) (width 0.25) (layer F.Cu) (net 14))
 (segment (start 159.575412 50.52) (end 157.315412 48.26) (width 0.25) (layer F.Cu) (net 14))
 (via (at 122.555 50.165) (size 0.8) (drill 0.4) (layers F.Cu B.Cu) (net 14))
 (segment (start 123.099999 49.620001) (end 122.555 50.165) (width 0.25) (layer B.Cu) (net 14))
 (segment (start 130.175 48.26) (end 128.814999 49.620001) (width 0.25) (layer B.Cu) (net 14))
 (segment (start 128.814999 49.620001) (end 123.099999 49.620001) (width 0.25) (layer B.Cu) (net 14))
 (segment (start 122.2 50.52) (end 120.3275 50.52) (width 0.25) (layer F.Cu) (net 14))
 (segment (start 122.555 50.165) (end 122.2 50.52) (width 0.25) (layer F.Cu) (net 14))
 (segment (start 112.39641 45.085) (end 95.885 45.085) (width 0.25) (layer F.Cu) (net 14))
 (segment (start 116.84141 49.53) (end 112.39641 45.085) (width 0.25) (layer F.Cu) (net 14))
 (segment (start 118.648942 49.53) (end 116.84141 49.53) (width 0.25) (layer F.Cu) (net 14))
 (segment (start 120.3275 50.52) (end 119.638942 50.52) (width 0.25) (layer F.Cu) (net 14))
 (segment (start 119.638942 50.52) (end 118.648942 49.53) (width 0.25) (layer F.Cu) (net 14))
 (via (at 128.27 50.619997) (size 0.8) (drill 0.4) (layers F.Cu B.Cu) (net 15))
 (segment (start 129.144998 49.744999) (end 128.27 50.619997) (width 0.25) (layer F.Cu) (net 15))
 (segment (start 158.164001 49.744999) (end 129.144998 49.744999) (width 0.25) (layer F.Cu) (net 15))
 (segment (start 160.9675 51.17) (end 159.589002 51.17) (width 0.25) (layer F.Cu) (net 15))
 (segment (start 159.589002 51.17) (end 158.164001 49.744999) (width 0.25) (layer F.Cu) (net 15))
 (via (at 122.555 51.435) (size 0.8) (drill 0.4) (layers F.Cu B.Cu) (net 15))
 (segment (start 128.27 50.619997) (end 123.370003 50.619997) (width 0.25) (layer B.Cu) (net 15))
 (segment (start 123.370003 50.619997) (end 122.555 51.435) (width 0.25) (layer B.Cu) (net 15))
 (segment (start 122.29 51.17) (end 120.3275 51.17) (width 0.25) (layer F.Cu) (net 15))
 (segment (start 122.555 51.435) (end 122.29 51.17) (width 0.25) (layer F.Cu) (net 15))
 (segment (start 114.3 47.625) (end 101.95001 47.625) (width 0.25) (layer F.Cu) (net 15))
 (segment (start 117.569999 50.894999) (end 114.3 47.625) (width 0.25) (layer F.Cu) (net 15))
 (segment (start 101.95001 47.625) (end 95.885 47.625) (width 0.25) (layer F.Cu) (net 15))
 (segment (start 118.674001 50.894999) (end 117.569999 50.894999) (width 0.25) (layer F.Cu) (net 15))
 (segment (start 120.3275 51.17) (end 118.949002 51.17) (width 0.25) (layer F.Cu) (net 15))
 (segment (start 118.949002 51.17) (end 118.674001 50.894999) (width 0.25) (layer F.Cu) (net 15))
 (via (at 164.465 46.355) (size 0.8) (drill 0.4) (layers F.Cu B.Cu) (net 16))
 (segment (start 164.214504 46.104504) (end 164.465 46.355) (width 0.25) (layer B.Cu) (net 16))
 (segment (start 152.77 47.025) (end 153.690496 46.104504) (width 0.25) (layer B.Cu) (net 16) (status 10))
 (segment (start 153.690496 46.104504) (end 164.214504 46.104504) (width 0.25) (layer B.Cu) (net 16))
 (segment (start 164.85 45.97) (end 166.6925 45.97) (width 0.25) (layer F.Cu) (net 16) (status 20))
 (segment (start 164.465 46.355) (end 164.85 45.97) (width 0.25) (layer F.Cu) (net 16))
 (via (at 158.589505 46.829505) (size 0.8) (drill 0.4) (layers F.Cu B.Cu) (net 17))
 (segment (start 154.57 47.025) (end 158.39401 47.025) (width 0.25) (layer B.Cu) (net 17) (status 10))
 (segment (start 158.39401 47.025) (end 158.589505 46.829505) (width 0.25) (layer B.Cu) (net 17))
 (segment (start 159.44901 45.97) (end 160.9675 45.97) (width 0.25) (layer F.Cu) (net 17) (status 20))
 (segment (start 158.589505 46.829505) (end 159.44901 45.97) (width 0.25) (layer F.Cu) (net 17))
 (via (at 158.75 48.26) (size 0.8) (drill 0.4) (layers F.Cu B.Cu) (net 18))
 (segment (start 154.57 48.225) (end 158.715 48.225) (width 0.25) (layer B.Cu) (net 18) (status 10))
 (segment (start 158.715 48.225) (end 158.75 48.26) (width 0.25) (layer B.Cu) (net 18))
 (segment (start 159.824315 46.62) (end 160.9675 46.62) (width 0.25) (layer F.Cu) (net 18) (status 20))
 (segment (start 158.75 47.694315) (end 159.824315 46.62) (width 0.25) (layer F.Cu) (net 18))
 (segment (start 158.75 48.26) (end 158.75 47.694315) (width 0.25) (layer F.Cu) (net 18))
 (via (at 168.91 46.355) (size 0.8) (drill 0.4) (layers F.Cu B.Cu) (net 19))
 (segment (start 174.89 48.225) (end 175.59 48.225) (width 0.25) (layer B.Cu) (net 19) (status 10))
 (segment (start 175.59 48.225) (end 175.665001 48.149999) (width 0.25) (layer B.Cu) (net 19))
 (segment (start 175.665001 48.149999) (end 175.665001 46.364999) (width 0.25) (layer B.Cu) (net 19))
 (segment (start 175.665001 46.364999) (end 175.149991 45.849989) (width 0.25) (layer B.Cu) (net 19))
 (segment (start 175.149991 45.849989) (end 169.415011 45.849989) (width 0.25) (layer B.Cu) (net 19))
 (segment (start 169.415011 45.849989) (end 168.91 46.355) (width 0.25) (layer B.Cu) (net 19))
 (segment (start 168.645 46.62) (end 166.6925 46.62) (width 0.25) (layer F.Cu) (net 19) (status 20))
 (segment (start 168.91 46.355) (end 168.645 46.62) (width 0.25) (layer F.Cu) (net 19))
 (via (at 168.91 47.625) (size 0.8) (drill 0.4) (layers F.Cu B.Cu) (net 20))
 (segment (start 170.235001 46.299999) (end 168.91 47.625) (width 0.25) (layer B.Cu) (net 20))
 (segment (start 174.89 47.025) (end 174.164999 46.299999) (width 0.25) (layer B.Cu) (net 20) (status 10))
 (segment (start 174.164999 46.299999) (end 170.235001 46.299999) (width 0.25) (layer B.Cu) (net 20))
 (segment (start 168.615 47.92) (end 166.6925 47.92) (width 0.25) (layer F.Cu) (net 20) (status 20))
 (segment (start 168.91 47.625) (end 168.615 47.92) (width 0.25) (layer F.Cu) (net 20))
 (via (at 168.91 48.895) (size 0.8) (drill 0.4) (layers F.Cu B.Cu) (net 21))
 (segment (start 173.09 47.025) (end 170.78 47.025) (width 0.25) (layer B.Cu) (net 21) (status 10))
 (segment (start 170.78 47.025) (end 168.91 48.895) (width 0.25) (layer B.Cu) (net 21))
 (segment (start 168.585 48.57) (end 166.6925 48.57) (width 0.25) (layer F.Cu) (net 21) (status 20))
 (segment (start 168.91 48.895) (end 168.585 48.57) (width 0.25) (layer F.Cu) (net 21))
 (segment (start 166.925 52.0525) (end 166.6925 51.82) (width 0.25) (layer F.Cu) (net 22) (status 20))
 (segment (start 166.925 53.975) (end 166.925 52.0525) (width 0.25) (layer F.Cu) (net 22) (status 10))
 (segment (start 174.204979 59.475021) (end 176.53 57.15) (width 0.25) (layer F.Cu) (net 5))
 (segment (start 101.385021 59.475021) (end 174.204979 59.475021) (width 0.25) (layer F.Cu) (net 5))
 (segment (start 100.33 58.42) (end 101.385021 59.475021) (width 0.25) (layer F.Cu) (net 5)))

